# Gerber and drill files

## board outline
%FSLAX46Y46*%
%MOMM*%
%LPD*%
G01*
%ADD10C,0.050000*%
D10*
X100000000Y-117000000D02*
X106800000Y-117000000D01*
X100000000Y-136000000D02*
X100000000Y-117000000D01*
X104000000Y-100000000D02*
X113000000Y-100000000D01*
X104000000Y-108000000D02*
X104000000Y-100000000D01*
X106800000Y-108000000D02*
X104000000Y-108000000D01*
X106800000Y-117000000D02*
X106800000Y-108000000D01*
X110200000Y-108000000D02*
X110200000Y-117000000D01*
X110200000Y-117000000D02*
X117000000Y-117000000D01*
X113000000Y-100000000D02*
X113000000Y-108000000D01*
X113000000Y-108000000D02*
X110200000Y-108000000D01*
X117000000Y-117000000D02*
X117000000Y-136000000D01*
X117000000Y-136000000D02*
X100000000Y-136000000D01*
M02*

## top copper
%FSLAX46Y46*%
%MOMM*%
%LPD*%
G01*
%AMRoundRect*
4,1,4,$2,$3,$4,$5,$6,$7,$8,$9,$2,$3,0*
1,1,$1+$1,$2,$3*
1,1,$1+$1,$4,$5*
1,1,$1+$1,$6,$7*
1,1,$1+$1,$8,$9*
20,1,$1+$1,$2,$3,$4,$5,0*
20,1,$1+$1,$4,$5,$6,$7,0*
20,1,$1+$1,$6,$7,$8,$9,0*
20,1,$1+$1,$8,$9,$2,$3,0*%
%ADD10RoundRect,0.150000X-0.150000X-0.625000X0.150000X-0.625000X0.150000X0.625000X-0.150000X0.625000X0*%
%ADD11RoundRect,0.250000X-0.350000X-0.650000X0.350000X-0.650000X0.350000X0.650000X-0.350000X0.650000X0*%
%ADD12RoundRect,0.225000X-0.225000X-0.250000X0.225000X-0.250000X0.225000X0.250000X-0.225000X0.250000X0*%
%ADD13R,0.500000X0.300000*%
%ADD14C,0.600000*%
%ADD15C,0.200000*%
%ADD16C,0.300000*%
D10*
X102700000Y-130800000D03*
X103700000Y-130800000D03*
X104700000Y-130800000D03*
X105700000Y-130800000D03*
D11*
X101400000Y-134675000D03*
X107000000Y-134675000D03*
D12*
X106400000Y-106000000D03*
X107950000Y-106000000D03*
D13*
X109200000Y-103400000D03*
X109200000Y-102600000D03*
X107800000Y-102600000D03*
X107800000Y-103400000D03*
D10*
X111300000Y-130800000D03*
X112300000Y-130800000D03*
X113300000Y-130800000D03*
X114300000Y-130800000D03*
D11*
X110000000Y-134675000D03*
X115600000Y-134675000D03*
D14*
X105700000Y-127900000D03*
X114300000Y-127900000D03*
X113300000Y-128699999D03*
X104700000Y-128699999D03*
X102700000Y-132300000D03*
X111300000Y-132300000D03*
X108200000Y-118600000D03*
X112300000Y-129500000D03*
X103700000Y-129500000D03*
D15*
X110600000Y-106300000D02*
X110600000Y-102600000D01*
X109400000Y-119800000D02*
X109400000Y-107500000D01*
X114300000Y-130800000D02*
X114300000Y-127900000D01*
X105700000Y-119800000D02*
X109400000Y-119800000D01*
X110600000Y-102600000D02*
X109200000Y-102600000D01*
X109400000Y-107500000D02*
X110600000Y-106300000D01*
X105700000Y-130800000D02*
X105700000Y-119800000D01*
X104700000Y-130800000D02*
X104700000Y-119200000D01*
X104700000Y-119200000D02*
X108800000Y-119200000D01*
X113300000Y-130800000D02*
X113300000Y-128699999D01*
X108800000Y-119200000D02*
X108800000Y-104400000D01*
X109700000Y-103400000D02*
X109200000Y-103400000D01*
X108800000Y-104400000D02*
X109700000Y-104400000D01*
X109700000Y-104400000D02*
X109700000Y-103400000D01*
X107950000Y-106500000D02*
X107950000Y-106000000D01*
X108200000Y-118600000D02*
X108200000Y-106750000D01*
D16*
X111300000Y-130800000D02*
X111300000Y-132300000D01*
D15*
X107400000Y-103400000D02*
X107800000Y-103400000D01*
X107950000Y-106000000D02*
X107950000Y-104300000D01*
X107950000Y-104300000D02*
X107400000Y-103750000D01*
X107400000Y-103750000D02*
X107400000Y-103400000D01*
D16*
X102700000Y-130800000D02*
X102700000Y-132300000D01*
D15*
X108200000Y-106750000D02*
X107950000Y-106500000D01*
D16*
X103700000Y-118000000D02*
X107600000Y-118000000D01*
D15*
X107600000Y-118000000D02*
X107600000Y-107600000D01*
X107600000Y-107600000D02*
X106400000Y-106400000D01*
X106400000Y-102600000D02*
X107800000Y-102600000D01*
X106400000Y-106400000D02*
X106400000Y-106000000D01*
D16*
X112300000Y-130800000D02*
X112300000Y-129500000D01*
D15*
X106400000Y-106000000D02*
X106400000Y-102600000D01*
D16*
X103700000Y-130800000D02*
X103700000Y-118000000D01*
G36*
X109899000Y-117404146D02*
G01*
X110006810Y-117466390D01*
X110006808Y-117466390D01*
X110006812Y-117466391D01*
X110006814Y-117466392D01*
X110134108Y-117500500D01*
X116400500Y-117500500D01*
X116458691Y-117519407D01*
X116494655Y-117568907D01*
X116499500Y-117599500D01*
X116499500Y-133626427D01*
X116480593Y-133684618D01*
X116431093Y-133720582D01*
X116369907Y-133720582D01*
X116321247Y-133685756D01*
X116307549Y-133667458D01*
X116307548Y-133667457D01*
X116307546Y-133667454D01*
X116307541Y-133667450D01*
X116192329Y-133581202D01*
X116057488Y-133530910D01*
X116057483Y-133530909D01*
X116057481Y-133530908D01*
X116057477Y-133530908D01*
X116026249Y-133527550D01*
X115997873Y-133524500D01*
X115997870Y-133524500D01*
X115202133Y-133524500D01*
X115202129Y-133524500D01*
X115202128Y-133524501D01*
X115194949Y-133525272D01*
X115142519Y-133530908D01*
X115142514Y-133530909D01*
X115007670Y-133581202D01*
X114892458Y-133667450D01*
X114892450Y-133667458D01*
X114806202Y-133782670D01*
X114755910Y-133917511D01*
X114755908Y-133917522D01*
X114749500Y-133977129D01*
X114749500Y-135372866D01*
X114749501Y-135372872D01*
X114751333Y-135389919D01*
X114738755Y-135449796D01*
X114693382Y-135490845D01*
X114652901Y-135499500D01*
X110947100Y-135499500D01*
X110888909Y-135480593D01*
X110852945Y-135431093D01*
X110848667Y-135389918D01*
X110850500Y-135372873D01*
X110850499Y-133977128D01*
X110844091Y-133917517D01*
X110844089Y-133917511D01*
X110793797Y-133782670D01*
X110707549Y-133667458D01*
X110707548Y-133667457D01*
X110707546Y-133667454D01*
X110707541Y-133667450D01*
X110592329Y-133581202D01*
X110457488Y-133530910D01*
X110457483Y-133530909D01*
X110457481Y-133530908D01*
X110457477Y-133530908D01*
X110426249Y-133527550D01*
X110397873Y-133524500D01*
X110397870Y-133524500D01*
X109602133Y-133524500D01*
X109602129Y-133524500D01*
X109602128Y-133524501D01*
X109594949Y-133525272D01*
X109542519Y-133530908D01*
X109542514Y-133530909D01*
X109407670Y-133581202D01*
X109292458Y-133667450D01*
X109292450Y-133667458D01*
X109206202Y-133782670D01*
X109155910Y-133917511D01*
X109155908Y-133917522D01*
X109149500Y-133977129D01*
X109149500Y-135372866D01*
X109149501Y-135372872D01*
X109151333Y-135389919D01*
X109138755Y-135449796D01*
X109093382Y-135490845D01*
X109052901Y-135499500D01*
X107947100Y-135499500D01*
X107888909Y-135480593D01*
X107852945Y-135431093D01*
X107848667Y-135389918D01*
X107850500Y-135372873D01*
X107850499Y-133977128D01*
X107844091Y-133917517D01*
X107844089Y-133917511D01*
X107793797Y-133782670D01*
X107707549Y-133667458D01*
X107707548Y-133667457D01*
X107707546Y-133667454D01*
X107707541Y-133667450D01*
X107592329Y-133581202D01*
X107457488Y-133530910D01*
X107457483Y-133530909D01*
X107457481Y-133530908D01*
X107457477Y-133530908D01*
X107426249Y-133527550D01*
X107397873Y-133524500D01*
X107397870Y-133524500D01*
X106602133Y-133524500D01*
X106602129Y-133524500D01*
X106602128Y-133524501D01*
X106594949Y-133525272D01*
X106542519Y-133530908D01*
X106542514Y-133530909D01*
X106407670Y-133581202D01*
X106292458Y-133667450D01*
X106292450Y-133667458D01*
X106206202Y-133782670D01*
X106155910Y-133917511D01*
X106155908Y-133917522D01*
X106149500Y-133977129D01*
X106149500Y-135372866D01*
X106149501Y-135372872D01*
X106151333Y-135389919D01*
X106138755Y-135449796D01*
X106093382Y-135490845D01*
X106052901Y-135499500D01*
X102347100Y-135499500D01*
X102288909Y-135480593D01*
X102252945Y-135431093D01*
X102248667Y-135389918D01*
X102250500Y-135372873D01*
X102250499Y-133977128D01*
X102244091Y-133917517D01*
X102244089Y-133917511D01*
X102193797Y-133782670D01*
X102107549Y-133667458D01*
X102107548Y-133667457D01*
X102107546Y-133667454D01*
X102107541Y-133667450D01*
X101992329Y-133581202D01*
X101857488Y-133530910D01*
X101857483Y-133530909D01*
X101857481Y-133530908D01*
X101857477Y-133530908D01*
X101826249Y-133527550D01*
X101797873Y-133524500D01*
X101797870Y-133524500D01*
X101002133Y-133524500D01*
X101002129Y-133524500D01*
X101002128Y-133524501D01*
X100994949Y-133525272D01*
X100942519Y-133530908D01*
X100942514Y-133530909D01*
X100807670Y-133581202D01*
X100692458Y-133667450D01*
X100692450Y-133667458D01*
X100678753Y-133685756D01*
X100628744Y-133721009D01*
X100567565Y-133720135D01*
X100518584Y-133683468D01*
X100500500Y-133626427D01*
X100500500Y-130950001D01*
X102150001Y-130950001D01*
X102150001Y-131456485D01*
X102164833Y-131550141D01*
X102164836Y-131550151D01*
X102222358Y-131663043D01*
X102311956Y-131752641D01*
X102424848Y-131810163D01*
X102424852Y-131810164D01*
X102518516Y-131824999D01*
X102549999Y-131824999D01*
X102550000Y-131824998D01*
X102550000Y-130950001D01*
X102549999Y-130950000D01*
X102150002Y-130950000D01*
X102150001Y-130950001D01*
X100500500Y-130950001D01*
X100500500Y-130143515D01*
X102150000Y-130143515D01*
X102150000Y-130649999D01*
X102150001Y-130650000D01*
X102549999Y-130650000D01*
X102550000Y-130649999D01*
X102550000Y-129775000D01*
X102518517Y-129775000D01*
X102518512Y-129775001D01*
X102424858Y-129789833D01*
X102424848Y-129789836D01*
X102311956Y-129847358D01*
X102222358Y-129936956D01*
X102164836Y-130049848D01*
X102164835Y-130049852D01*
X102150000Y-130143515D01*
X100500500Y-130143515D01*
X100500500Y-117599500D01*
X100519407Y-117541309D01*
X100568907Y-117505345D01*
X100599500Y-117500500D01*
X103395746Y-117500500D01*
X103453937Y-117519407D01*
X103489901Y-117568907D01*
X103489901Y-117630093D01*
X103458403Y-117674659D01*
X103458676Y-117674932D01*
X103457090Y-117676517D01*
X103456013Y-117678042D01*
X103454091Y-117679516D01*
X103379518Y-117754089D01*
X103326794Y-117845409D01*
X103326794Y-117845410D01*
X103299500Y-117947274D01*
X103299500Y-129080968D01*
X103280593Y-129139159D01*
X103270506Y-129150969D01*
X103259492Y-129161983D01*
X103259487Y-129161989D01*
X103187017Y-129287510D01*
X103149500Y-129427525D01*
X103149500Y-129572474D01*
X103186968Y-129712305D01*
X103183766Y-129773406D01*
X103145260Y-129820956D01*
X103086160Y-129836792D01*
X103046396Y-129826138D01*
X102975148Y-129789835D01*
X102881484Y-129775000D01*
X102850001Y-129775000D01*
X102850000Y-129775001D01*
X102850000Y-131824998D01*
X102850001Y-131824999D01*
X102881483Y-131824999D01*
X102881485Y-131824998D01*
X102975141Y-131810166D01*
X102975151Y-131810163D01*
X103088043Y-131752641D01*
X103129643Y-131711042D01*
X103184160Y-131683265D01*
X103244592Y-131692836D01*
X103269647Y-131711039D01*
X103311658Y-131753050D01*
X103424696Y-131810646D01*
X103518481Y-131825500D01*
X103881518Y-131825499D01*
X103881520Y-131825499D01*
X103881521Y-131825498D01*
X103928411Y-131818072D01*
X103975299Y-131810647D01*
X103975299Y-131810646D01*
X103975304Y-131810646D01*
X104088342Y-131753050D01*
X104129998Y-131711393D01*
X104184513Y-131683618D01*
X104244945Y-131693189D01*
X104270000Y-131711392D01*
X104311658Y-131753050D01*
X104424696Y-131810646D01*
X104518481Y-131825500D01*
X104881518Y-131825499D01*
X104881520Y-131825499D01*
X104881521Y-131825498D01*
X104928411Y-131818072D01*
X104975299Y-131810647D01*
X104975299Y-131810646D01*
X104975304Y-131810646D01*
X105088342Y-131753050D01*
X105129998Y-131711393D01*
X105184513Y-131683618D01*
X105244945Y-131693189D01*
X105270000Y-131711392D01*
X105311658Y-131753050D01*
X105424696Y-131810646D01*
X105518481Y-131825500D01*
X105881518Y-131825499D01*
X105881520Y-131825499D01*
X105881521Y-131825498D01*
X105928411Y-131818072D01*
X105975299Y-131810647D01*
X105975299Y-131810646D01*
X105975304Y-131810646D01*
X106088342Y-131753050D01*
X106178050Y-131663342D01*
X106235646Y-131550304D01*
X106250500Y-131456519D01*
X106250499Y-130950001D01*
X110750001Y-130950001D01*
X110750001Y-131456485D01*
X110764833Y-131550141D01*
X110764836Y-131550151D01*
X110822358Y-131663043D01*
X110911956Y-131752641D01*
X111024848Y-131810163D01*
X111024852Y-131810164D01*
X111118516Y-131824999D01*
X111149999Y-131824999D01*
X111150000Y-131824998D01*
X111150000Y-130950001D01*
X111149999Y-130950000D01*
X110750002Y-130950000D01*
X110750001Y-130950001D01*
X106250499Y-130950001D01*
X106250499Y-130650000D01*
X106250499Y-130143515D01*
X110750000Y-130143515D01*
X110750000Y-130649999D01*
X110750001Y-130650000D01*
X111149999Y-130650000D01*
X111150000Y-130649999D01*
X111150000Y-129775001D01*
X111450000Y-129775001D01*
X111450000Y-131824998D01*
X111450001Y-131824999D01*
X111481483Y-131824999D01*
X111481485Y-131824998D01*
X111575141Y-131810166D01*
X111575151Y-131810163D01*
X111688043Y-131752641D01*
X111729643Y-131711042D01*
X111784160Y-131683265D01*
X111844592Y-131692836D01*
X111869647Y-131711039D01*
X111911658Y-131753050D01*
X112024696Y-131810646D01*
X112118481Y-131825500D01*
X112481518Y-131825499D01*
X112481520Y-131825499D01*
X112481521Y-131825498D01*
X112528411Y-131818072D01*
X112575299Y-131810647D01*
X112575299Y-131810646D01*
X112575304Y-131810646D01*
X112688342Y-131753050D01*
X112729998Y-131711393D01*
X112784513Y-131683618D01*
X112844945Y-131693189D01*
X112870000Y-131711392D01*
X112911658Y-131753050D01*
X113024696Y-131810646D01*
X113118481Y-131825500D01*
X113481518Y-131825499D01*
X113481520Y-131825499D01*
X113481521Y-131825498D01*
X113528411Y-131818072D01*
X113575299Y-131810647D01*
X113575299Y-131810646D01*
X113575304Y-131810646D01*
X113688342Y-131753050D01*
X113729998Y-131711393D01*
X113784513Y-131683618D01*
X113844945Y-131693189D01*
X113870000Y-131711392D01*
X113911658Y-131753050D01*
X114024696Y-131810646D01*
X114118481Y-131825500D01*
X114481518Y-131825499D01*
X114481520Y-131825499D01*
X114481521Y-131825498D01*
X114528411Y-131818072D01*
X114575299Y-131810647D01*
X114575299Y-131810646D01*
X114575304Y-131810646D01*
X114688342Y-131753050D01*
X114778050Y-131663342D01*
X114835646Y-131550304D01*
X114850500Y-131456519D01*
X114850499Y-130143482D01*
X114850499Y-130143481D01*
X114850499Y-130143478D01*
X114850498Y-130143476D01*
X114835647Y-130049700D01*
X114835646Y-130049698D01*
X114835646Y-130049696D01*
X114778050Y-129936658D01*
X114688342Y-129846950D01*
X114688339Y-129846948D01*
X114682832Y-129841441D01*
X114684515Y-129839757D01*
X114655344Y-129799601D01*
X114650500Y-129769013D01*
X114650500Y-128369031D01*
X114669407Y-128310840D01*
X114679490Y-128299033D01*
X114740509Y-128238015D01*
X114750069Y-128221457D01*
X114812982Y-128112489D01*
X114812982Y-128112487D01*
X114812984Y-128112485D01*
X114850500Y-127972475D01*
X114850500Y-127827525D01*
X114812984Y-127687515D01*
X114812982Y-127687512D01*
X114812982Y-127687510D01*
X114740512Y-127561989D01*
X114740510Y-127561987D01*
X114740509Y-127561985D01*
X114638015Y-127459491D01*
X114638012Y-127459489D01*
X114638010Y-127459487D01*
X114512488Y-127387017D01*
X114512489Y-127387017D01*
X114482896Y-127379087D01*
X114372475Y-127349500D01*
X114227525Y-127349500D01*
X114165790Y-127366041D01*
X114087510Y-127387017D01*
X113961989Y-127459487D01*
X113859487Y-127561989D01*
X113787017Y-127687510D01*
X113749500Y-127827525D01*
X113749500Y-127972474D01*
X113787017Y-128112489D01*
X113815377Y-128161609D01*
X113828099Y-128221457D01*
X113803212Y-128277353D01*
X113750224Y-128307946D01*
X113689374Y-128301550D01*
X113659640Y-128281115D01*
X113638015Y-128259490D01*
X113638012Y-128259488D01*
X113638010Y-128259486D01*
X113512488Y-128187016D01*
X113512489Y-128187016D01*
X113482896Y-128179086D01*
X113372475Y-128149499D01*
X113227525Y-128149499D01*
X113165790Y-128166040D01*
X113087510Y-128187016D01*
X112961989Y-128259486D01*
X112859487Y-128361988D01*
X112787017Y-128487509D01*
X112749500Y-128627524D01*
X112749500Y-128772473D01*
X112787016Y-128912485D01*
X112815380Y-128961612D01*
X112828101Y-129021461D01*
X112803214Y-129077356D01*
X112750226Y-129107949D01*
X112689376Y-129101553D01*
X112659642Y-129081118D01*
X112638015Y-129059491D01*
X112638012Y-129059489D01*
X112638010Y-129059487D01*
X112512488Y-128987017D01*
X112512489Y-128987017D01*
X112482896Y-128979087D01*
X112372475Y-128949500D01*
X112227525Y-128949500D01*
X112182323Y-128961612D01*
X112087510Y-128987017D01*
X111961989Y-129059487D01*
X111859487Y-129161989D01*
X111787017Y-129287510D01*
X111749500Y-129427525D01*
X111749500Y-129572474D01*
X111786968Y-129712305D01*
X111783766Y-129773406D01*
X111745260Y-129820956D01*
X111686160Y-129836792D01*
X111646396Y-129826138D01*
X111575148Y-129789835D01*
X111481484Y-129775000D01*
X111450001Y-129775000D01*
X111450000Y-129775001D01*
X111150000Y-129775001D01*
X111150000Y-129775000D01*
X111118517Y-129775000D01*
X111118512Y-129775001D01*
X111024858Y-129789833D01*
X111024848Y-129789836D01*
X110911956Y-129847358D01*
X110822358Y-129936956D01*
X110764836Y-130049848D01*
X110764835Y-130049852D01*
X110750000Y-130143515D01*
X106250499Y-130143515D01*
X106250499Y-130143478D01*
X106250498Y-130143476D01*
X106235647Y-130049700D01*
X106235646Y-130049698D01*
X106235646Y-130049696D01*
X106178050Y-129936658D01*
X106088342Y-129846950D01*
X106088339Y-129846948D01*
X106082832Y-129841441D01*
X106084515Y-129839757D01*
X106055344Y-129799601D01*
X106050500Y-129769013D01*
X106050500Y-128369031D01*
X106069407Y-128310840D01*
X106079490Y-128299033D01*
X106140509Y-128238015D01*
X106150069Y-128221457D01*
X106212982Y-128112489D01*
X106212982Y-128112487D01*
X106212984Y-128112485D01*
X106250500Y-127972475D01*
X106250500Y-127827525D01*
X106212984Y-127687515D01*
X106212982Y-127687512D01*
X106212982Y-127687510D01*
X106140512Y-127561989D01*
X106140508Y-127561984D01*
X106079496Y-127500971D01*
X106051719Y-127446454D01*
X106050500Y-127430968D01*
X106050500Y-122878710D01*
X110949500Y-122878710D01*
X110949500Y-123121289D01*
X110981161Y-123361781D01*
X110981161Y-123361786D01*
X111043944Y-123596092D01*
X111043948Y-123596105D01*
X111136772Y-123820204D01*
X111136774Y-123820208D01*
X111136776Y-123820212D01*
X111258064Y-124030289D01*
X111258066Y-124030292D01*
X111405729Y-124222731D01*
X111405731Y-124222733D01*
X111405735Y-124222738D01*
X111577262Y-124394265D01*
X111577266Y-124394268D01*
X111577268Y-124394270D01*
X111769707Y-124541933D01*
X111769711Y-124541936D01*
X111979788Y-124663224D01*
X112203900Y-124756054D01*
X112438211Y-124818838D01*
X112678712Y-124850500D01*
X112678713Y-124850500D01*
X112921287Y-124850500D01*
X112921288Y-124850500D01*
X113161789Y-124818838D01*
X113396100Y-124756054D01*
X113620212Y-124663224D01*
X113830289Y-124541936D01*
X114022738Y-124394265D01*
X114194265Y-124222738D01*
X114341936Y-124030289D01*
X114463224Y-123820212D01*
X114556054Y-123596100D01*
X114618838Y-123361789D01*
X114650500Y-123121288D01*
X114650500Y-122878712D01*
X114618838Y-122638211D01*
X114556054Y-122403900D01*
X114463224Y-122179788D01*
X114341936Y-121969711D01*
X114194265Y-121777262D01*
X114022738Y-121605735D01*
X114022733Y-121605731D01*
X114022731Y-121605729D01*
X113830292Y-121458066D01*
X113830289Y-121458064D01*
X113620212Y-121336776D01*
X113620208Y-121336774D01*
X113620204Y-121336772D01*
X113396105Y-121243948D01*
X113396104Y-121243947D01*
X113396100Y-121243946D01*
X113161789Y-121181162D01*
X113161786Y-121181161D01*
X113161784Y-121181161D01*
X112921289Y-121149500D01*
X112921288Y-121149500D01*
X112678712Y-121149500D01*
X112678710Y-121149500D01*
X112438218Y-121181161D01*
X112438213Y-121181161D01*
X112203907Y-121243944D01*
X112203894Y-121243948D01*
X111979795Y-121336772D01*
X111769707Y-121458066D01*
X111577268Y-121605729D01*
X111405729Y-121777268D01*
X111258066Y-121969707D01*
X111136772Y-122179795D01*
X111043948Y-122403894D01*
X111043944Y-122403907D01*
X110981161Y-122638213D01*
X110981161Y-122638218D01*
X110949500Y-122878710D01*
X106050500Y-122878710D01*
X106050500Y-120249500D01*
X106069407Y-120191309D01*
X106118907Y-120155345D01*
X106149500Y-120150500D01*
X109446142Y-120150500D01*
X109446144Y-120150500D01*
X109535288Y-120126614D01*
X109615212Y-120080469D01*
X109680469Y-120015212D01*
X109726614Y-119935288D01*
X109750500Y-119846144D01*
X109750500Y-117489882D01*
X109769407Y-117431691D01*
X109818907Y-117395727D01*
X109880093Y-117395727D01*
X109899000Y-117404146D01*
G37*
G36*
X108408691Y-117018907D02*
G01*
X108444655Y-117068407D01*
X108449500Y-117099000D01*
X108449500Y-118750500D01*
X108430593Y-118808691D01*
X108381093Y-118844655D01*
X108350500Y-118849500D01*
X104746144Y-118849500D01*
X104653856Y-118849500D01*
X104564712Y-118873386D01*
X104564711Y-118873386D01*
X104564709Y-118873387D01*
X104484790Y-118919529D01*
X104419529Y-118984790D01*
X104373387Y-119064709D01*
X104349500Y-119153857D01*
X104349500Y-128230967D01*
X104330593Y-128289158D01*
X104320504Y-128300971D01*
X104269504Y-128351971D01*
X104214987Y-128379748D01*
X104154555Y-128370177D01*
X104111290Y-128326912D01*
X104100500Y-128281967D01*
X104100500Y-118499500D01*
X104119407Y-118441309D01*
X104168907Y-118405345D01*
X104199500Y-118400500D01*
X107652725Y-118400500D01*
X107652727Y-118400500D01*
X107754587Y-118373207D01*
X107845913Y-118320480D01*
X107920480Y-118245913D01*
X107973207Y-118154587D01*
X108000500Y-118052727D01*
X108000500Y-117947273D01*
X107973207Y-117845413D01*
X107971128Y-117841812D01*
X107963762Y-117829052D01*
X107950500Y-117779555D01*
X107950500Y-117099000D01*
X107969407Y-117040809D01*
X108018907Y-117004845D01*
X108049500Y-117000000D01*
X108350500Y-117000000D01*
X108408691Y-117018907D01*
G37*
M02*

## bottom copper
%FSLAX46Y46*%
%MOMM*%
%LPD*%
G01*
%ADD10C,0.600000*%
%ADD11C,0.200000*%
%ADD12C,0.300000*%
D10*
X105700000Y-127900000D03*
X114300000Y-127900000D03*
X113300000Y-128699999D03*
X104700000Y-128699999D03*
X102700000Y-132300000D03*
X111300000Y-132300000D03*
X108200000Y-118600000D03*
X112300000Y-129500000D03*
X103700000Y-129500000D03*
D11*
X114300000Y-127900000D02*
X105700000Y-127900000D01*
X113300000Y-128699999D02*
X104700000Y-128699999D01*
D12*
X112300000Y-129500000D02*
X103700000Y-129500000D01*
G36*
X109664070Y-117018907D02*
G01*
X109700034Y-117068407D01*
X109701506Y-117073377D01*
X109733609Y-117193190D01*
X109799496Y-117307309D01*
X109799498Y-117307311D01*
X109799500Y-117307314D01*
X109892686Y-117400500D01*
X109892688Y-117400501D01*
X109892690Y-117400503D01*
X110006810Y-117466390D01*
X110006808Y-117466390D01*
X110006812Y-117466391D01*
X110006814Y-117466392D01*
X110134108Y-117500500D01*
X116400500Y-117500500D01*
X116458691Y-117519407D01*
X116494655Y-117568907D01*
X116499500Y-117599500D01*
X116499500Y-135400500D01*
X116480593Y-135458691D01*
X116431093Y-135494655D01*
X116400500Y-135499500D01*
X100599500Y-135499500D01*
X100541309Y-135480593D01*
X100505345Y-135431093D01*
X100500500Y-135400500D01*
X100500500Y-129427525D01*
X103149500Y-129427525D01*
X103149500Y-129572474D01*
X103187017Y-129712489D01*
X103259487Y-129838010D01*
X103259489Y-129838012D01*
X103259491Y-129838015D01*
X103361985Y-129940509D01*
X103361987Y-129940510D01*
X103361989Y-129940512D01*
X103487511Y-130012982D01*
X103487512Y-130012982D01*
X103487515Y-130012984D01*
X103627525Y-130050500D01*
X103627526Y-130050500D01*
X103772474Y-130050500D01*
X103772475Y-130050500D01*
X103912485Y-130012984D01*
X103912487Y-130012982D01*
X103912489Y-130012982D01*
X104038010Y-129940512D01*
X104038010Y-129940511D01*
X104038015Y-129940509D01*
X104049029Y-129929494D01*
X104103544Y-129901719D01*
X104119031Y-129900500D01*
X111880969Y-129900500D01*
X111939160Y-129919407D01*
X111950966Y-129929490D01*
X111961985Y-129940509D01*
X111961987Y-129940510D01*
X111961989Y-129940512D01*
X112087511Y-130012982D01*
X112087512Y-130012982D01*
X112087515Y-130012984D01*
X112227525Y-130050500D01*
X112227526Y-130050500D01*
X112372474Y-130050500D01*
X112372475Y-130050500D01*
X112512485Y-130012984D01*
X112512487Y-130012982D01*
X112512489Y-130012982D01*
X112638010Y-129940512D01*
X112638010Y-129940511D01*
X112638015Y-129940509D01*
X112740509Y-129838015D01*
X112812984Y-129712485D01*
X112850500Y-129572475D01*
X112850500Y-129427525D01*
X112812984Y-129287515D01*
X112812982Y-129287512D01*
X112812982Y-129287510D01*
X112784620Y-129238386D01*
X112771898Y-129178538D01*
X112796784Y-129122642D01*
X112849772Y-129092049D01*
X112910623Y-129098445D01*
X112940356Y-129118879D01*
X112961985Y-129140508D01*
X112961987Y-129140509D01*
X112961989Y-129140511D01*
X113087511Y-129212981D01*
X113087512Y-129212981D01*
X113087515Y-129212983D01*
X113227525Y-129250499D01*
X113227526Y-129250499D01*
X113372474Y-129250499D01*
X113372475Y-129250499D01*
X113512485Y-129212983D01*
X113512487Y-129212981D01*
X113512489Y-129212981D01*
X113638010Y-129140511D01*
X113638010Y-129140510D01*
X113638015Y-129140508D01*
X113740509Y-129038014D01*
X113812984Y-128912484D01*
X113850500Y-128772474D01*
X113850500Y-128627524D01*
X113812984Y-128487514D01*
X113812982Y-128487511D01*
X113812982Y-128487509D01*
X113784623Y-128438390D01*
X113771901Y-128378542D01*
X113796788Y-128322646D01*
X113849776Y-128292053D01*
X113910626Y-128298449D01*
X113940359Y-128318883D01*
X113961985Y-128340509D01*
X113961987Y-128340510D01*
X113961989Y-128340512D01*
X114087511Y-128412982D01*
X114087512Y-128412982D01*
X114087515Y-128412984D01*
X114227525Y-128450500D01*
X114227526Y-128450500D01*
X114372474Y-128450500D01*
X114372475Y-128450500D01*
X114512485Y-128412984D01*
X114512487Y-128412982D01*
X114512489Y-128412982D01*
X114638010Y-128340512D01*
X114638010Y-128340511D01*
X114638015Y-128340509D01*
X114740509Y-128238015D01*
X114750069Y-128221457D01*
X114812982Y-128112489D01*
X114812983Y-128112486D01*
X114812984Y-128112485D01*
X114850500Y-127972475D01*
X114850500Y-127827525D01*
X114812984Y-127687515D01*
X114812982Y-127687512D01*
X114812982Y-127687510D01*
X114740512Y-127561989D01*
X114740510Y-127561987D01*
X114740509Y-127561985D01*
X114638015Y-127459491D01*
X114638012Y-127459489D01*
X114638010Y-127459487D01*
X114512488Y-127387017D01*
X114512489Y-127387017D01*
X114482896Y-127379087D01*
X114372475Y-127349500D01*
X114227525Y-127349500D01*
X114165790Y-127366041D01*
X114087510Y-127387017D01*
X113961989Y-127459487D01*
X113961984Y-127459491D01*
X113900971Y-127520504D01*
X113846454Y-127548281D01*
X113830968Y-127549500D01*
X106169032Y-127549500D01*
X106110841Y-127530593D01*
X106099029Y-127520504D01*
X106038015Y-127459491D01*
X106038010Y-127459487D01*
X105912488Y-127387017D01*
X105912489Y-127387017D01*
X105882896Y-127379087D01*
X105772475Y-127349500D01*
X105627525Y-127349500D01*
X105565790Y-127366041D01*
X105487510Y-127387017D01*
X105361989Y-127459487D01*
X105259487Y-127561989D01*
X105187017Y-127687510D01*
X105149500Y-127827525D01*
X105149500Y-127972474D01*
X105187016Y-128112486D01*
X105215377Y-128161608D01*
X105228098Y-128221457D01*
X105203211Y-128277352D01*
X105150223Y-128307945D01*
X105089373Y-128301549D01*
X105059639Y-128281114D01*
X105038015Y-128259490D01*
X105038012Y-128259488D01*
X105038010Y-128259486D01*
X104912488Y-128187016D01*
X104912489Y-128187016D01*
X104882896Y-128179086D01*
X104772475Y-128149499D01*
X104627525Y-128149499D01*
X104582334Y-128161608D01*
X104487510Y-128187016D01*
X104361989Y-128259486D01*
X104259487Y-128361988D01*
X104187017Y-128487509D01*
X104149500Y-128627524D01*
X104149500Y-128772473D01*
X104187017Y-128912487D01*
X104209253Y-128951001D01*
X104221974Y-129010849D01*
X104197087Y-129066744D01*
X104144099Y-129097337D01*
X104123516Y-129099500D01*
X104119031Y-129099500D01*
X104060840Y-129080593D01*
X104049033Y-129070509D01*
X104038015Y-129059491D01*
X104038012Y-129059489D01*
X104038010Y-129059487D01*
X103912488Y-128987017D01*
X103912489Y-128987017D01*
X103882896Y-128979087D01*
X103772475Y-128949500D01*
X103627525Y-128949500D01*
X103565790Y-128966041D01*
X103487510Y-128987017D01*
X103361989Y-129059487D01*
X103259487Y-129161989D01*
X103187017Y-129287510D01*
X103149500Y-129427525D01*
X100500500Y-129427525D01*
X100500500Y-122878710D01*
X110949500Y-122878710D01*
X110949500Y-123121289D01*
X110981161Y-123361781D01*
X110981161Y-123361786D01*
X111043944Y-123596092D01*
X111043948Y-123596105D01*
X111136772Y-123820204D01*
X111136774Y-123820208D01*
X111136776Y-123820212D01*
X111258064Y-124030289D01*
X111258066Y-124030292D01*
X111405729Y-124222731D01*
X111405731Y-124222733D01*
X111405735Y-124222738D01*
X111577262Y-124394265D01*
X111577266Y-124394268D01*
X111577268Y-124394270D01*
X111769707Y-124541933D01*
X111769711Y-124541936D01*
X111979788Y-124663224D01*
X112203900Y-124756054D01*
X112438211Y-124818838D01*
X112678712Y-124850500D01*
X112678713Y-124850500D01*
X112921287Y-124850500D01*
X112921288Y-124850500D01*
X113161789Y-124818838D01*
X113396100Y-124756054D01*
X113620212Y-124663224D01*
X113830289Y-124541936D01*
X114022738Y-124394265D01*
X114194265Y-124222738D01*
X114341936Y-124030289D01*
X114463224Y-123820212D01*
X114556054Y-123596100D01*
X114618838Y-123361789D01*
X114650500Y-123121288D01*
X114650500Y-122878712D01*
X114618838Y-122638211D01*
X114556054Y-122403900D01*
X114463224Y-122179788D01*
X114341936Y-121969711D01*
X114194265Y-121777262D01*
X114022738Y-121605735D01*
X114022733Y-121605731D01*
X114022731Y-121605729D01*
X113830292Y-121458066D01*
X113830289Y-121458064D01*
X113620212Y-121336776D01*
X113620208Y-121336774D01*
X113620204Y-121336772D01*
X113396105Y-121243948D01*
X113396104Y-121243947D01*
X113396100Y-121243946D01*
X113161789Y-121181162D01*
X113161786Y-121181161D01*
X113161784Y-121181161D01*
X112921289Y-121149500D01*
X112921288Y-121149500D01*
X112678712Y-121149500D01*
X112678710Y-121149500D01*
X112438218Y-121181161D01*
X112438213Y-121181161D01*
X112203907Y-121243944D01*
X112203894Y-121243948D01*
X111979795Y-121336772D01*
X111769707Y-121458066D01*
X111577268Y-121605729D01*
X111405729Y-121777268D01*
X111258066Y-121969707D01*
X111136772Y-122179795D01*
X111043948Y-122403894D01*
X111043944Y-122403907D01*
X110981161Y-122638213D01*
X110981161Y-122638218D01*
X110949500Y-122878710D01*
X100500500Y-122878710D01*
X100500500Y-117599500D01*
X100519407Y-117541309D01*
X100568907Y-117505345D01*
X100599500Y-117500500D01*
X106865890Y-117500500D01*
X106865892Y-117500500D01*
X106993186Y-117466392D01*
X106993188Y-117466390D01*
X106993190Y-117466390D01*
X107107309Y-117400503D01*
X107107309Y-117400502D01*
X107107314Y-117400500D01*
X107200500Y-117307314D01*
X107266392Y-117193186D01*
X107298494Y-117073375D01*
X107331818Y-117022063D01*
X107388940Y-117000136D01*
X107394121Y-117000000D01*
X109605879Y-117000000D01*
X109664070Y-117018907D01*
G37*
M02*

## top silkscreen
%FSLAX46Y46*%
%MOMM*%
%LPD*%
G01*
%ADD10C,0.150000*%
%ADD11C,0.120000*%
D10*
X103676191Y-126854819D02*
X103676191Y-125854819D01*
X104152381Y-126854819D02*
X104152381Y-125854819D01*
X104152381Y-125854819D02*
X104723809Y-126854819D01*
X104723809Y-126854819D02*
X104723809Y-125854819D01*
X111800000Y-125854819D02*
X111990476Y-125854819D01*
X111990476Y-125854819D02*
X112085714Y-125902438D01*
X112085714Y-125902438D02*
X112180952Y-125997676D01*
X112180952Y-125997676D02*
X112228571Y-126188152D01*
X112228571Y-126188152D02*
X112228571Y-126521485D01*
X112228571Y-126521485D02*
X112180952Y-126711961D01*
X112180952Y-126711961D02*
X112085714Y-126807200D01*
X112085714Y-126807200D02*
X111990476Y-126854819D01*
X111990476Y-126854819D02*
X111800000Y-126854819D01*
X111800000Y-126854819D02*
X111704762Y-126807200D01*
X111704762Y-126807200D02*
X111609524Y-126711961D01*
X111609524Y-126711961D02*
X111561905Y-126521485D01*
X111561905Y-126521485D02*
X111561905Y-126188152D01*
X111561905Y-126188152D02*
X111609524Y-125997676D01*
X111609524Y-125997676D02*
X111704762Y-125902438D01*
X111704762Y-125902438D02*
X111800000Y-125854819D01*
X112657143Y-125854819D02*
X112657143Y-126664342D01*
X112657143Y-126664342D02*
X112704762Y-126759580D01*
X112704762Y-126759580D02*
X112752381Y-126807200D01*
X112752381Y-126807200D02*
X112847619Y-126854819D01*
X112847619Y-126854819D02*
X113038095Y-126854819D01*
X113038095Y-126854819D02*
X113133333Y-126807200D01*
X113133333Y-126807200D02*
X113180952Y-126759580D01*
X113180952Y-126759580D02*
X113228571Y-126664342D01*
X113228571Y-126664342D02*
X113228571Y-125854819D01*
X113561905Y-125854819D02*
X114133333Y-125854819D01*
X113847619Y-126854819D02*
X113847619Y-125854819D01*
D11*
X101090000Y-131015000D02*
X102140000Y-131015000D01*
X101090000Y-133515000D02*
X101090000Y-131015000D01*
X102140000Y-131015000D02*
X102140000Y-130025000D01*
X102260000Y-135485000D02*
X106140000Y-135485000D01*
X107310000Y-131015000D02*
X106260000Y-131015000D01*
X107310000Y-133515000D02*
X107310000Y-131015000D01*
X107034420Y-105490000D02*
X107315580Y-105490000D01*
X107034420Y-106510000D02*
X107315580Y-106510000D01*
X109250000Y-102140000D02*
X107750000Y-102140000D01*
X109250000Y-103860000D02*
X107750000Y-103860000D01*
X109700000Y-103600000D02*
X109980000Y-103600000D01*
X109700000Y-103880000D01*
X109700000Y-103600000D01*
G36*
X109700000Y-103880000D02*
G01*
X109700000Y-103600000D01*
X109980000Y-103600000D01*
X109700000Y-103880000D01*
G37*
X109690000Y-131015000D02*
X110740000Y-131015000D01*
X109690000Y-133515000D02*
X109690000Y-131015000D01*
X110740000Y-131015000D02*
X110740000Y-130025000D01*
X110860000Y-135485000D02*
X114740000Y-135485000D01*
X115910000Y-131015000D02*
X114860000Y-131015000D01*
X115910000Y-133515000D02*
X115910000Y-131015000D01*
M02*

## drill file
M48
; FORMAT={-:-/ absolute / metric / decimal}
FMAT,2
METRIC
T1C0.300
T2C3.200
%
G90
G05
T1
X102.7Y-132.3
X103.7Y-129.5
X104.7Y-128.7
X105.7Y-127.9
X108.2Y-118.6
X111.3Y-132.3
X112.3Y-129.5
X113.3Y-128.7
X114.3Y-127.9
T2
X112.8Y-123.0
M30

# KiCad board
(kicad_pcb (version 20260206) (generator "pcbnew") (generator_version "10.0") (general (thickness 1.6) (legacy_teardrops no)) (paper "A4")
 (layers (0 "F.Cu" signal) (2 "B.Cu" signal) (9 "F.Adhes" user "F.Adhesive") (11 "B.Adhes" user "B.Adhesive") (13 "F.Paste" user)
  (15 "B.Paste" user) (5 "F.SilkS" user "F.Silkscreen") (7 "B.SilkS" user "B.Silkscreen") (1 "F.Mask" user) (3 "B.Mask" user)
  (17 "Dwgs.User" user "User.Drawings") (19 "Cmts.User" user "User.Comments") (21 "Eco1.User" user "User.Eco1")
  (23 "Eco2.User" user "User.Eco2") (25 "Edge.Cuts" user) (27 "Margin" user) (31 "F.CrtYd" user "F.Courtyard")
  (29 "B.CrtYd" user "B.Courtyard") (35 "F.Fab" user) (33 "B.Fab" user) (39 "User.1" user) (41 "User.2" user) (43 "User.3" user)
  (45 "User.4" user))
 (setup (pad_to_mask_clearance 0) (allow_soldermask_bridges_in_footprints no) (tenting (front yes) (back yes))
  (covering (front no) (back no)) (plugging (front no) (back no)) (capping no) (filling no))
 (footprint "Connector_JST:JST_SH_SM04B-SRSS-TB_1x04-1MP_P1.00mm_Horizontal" (layer "F.Cu") (at 104.2 132.8)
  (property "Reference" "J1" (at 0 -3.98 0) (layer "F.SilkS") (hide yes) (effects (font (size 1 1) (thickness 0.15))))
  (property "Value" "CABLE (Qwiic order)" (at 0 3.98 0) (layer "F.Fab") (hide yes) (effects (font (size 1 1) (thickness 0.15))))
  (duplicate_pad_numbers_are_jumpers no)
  (fp_line (start -3.11 -1.785) (end -2.06 -1.785) (stroke (width 0.12) (type solid)) (layer "F.SilkS"))
  (fp_line (start -3.11 0.715) (end -3.11 -1.785) (stroke (width 0.12) (type solid)) (layer "F.SilkS"))
  (fp_line (start -2.06 -1.785) (end -2.06 -2.775) (stroke (width 0.12) (type solid)) (layer "F.SilkS"))
  (fp_line (start -1.94 2.685) (end 1.94 2.685) (stroke (width 0.12) (type solid)) (layer "F.SilkS"))
  (fp_line (start 3.11 -1.785) (end 2.06 -1.785) (stroke (width 0.12) (type solid)) (layer "F.SilkS"))
  (fp_line (start 3.11 0.715) (end 3.11 -1.785) (stroke (width 0.12) (type solid)) (layer "F.SilkS"))
  (pad "1" smd roundrect (at -1.5 -2) (size 0.6 1.55) (layers "F.Cu" "F.Mask" "F.Paste") (roundrect_rratio 0.25) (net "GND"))
  (pad "2" smd roundrect (at -0.5 -2) (size 0.6 1.55) (layers "F.Cu" "F.Mask" "F.Paste") (roundrect_rratio 0.25) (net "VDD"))
  (pad "3" smd roundrect (at 0.5 -2) (size 0.6 1.55) (layers "F.Cu" "F.Mask" "F.Paste") (roundrect_rratio 0.25) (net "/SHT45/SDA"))
  (pad "4" smd roundrect (at 1.5 -2) (size 0.6 1.55) (layers "F.Cu" "F.Mask" "F.Paste") (roundrect_rratio 0.25) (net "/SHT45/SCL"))
  (pad "MP" smd roundrect (at -2.8 1.875) (size 1.2 1.8) (layers "F.Cu" "F.Mask" "F.Paste") (roundrect_rratio 0.208333))
  (pad "MP" smd roundrect (at 2.8 1.875) (size 1.2 1.8) (layers "F.Cu" "F.Mask" "F.Paste") (roundrect_rratio 0.208333)))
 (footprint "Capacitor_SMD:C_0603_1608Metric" (layer "F.Cu") (at 107.175 106)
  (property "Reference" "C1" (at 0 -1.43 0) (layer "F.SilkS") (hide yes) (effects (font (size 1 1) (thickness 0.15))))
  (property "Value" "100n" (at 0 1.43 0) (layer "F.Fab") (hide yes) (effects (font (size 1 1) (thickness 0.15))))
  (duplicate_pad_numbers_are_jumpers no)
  (fp_line (start -0.14058 -0.51) (end 0.14058 -0.51) (stroke (width 0.12) (type solid)) (layer "F.SilkS"))
  (fp_line (start -0.14058 0.51) (end 0.14058 0.51) (stroke (width 0.12) (type solid)) (layer "F.SilkS"))
  (pad "1" smd roundrect (at -0.775 0) (size 0.9 0.95) (layers "F.Cu" "F.Mask" "F.Paste") (roundrect_rratio 0.25) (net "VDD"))
  (pad "2" smd roundrect (at 0.775 0) (size 0.9 0.95) (layers "F.Cu" "F.Mask" "F.Paste") (roundrect_rratio 0.25) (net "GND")))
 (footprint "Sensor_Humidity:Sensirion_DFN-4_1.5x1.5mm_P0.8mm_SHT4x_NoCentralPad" (layer "F.Cu") (at 108.5 103 180)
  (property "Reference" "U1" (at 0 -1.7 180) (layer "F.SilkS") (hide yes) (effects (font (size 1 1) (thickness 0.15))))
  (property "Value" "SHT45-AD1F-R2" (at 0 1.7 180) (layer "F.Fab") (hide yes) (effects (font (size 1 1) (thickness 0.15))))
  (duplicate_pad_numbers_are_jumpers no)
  (fp_line (start -0.75 0.86) (end 0.75 0.86) (stroke (width 0.12) (type solid)) (layer "F.SilkS"))
  (fp_line (start -0.75 -0.86) (end 0.75 -0.86) (stroke (width 0.12) (type solid)) (layer "F.SilkS"))
  (fp_poly
   (pts (xy -1.2 -0.6) (xy -1.48 -0.6) (xy -1.2 -0.88) (xy -1.2 -0.6)) (stroke (width 0.12) (type solid)) (fill yes) (layer "F.SilkS"))
  (pad "1" smd rect (at -0.7 -0.4 180) (size 0.5 0.3) (layers "F.Cu" "F.Mask" "F.Paste") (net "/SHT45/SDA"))
  (pad "2" smd rect (at -0.7 0.4 180) (size 0.5 0.3) (layers "F.Cu" "F.Mask" "F.Paste") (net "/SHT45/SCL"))
  (pad "3" smd rect (at 0.7 0.4 180) (size 0.5 0.3) (layers "F.Cu" "F.Mask" "F.Paste") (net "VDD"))
  (pad "4" smd rect (at 0.7 -0.4 180) (size 0.5 0.3) (layers "F.Cu" "F.Mask" "F.Paste") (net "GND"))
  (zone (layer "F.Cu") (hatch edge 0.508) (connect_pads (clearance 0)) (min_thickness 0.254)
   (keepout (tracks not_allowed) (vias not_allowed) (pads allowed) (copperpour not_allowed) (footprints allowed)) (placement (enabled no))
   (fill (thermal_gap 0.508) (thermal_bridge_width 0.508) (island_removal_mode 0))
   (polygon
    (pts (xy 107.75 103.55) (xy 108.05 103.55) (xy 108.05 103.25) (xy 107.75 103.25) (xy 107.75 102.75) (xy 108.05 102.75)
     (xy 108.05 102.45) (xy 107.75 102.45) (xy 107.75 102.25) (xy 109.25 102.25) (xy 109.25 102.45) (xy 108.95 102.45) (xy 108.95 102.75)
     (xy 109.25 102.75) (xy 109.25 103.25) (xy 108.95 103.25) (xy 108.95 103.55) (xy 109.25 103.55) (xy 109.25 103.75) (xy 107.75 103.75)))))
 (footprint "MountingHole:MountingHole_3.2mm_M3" (layer "F.Cu") (at 112.8 123)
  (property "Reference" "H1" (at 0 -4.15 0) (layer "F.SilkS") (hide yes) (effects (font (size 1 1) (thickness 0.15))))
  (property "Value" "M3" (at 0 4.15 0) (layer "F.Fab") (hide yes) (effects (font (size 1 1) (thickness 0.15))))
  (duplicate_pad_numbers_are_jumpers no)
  (pad "" np_thru_hole circle (at 0 0) (size 3.2 3.2) (drill 3.2) (layers "*.Cu" "*.Mask")))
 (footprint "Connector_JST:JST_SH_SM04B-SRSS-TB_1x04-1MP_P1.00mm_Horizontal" (layer "F.Cu") (at 112.8 132.8)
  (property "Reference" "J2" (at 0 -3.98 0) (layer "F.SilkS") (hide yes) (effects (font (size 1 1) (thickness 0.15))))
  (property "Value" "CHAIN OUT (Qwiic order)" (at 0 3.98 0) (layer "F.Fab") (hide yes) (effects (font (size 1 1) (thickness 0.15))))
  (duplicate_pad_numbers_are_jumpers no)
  (fp_line (start -3.11 -1.785) (end -2.06 -1.785) (stroke (width 0.12) (type solid)) (layer "F.SilkS"))
  (fp_line (start -3.11 0.715) (end -3.11 -1.785) (stroke (width 0.12) (type solid)) (layer "F.SilkS"))
  (fp_line (start -2.06 -1.785) (end -2.06 -2.775) (stroke (width 0.12) (type solid)) (layer "F.SilkS"))
  (fp_line (start -1.94 2.685) (end 1.94 2.685) (stroke (width 0.12) (type solid)) (layer "F.SilkS"))
  (fp_line (start 3.11 -1.785) (end 2.06 -1.785) (stroke (width 0.12) (type solid)) (layer "F.SilkS"))
  (fp_line (start 3.11 0.715) (end 3.11 -1.785) (stroke (width 0.12) (type solid)) (layer "F.SilkS"))
  (pad "1" smd roundrect (at -1.5 -2) (size 0.6 1.55) (layers "F.Cu" "F.Mask" "F.Paste") (roundrect_rratio 0.25) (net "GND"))
  (pad "2" smd roundrect (at -0.5 -2) (size 0.6 1.55) (layers "F.Cu" "F.Mask" "F.Paste") (roundrect_rratio 0.25) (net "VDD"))
  (pad "3" smd roundrect (at 0.5 -2) (size 0.6 1.55) (layers "F.Cu" "F.Mask" "F.Paste") (roundrect_rratio 0.25) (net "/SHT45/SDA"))
  (pad "4" smd roundrect (at 1.5 -2) (size 0.6 1.55) (layers "F.Cu" "F.Mask" "F.Paste") (roundrect_rratio 0.25) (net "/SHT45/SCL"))
  (pad "MP" smd roundrect (at -2.8 1.875) (size 1.2 1.8) (layers "F.Cu" "F.Mask" "F.Paste") (roundrect_rratio 0.208333))
  (pad "MP" smd roundrect (at 2.8 1.875) (size 1.2 1.8) (layers "F.Cu" "F.Mask" "F.Paste") (roundrect_rratio 0.208333)))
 (gr_line (start 100 117) (end 106.8 117) (stroke (width 0.05) (type default)) (layer "Edge.Cuts"))
 (gr_line (start 100 136) (end 100 117) (stroke (width 0.05) (type default)) (layer "Edge.Cuts"))
 (gr_line (start 104 100) (end 113 100) (stroke (width 0.05) (type default)) (layer "Edge.Cuts"))
 (gr_line (start 104 108) (end 104 100) (stroke (width 0.05) (type default)) (layer "Edge.Cuts"))
 (gr_line (start 106.8 108) (end 104 108) (stroke (width 0.05) (type default)) (layer "Edge.Cuts"))
 (gr_line (start 106.8 117) (end 106.8 108) (stroke (width 0.05) (type default)) (layer "Edge.Cuts"))
 (gr_line (start 110.2 108) (end 110.2 117) (stroke (width 0.05) (type default)) (layer "Edge.Cuts"))
 (gr_line (start 110.2 117) (end 117 117) (stroke (width 0.05) (type default)) (layer "Edge.Cuts"))
 (gr_line (start 113 100) (end 113 108) (stroke (width 0.05) (type default)) (layer "Edge.Cuts"))
 (gr_line (start 113 108) (end 110.2 108) (stroke (width 0.05) (type default)) (layer "Edge.Cuts"))
 (gr_line (start 117 117) (end 117 136) (stroke (width 0.05) (type default)) (layer "Edge.Cuts"))
 (gr_line (start 117 136) (end 100 136) (stroke (width 0.05) (type default)) (layer "Edge.Cuts"))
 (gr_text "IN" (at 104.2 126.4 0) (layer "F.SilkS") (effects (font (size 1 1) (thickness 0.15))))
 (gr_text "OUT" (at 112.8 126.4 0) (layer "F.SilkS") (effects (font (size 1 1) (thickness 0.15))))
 (segment (start 110.6 106.3) (end 110.6 102.6) (width 0.2) (layer "F.Cu") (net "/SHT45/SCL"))
 (segment (start 109.4 119.8) (end 109.4 107.5) (width 0.2) (layer "F.Cu") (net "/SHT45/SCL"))
 (segment (start 114.3 130.8) (end 114.3 127.9) (width 0.2) (layer "F.Cu") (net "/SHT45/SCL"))
 (segment (start 105.7 119.8) (end 109.4 119.8) (width 0.2) (layer "F.Cu") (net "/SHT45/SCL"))
 (segment (start 110.6 102.6) (end 109.2 102.6) (width 0.2) (layer "F.Cu") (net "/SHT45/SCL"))
 (segment (start 109.4 107.5) (end 110.6 106.3) (width 0.2) (layer "F.Cu") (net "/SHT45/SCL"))
 (segment (start 105.7 130.8) (end 105.7 119.8) (width 0.2) (layer "F.Cu") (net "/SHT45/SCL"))
 (via (at 105.7 127.9) (size 0.6) (drill 0.3) (layers "F.Cu" "B.Cu") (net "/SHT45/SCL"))
 (via (at 114.3 127.9) (size 0.6) (drill 0.3) (layers "F.Cu" "B.Cu") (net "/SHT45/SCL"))
 (segment (start 114.3 127.9) (end 105.7 127.9) (width 0.2) (layer "B.Cu") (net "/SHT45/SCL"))
 (segment (start 104.7 130.8) (end 104.7 119.2) (width 0.2) (layer "F.Cu") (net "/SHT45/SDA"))
 (segment (start 104.7 119.2) (end 108.8 119.2) (width 0.2) (layer "F.Cu") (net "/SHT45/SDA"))
 (segment (start 113.3 130.8) (end 113.3 128.699999) (width 0.2) (layer "F.Cu") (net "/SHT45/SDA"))
 (segment (start 108.8 119.2) (end 108.8 104.4) (width 0.2) (layer "F.Cu") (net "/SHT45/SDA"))
 (segment (start 109.7 103.4) (end 109.2 103.4) (width 0.2) (layer "F.Cu") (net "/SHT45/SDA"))
 (segment (start 108.8 104.4) (end 109.7 104.4) (width 0.2) (layer "F.Cu") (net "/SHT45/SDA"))
 (segment (start 109.7 104.4) (end 109.7 103.4) (width 0.2) (layer "F.Cu") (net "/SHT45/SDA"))
 (via (at 113.3 128.699999) (size 0.6) (drill 0.3) (layers "F.Cu" "B.Cu") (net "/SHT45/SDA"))
 (via (at 104.7 128.699999) (size 0.6) (drill 0.3) (layers "F.Cu" "B.Cu") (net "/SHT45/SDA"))
 (segment (start 113.3 128.699999) (end 104.7 128.699999) (width 0.2) (layer "B.Cu") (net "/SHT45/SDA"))
 (segment (start 107.95 106.5) (end 107.95 106) (width 0.2) (layer "F.Cu") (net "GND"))
 (segment (start 108.2 118.6) (end 108.2 106.75) (width 0.2) (layer "F.Cu") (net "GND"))
 (segment (start 111.3 130.8) (end 111.3 132.3) (width 0.3) (layer "F.Cu") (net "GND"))
 (segment (start 107.4 103.4) (end 107.8 103.4) (width 0.2) (layer "F.Cu") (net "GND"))
 (segment (start 107.95 106) (end 107.95 104.3) (width 0.2) (layer "F.Cu") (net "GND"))
 (segment (start 107.95 104.3) (end 107.4 103.75) (width 0.2) (layer "F.Cu") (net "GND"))
 (segment (start 107.4 103.75) (end 107.4 103.4) (width 0.2) (layer "F.Cu") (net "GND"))
 (segment (start 102.7 130.8) (end 102.7 132.3) (width 0.3) (layer "F.Cu") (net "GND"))
 (segment (start 108.2 106.75) (end 107.95 106.5) (width 0.2) (layer "F.Cu") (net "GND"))
 (via (at 102.7 132.3) (size 0.6) (drill 0.3) (layers "F.Cu" "B.Cu") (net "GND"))
 (via (at 111.3 132.3) (size 0.6) (drill 0.3) (layers "F.Cu" "B.Cu") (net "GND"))
 (via (at 108.2 118.6) (size 0.6) (drill 0.3) (layers "F.Cu" "B.Cu") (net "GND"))
 (segment (start 103.7 118) (end 107.6 118) (width 0.3) (layer "F.Cu") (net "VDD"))
 (segment (start 107.6 118) (end 107.6 107.6) (width 0.2) (layer "F.Cu") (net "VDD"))
 (segment (start 107.6 107.6) (end 106.4 106.4) (width 0.2) (layer "F.Cu") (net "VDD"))
 (segment (start 106.4 102.6) (end 107.8 102.6) (width 0.2) (layer "F.Cu") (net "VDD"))
 (segment (start 106.4 106.4) (end 106.4 106) (width 0.2) (layer "F.Cu") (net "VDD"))
 (segment (start 112.3 130.8) (end 112.3 129.5) (width 0.3) (layer "F.Cu") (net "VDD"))
 (segment (start 106.4 106) (end 106.4 102.6) (width 0.2) (layer "F.Cu") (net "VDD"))
 (segment (start 103.7 130.8) (end 103.7 118) (width 0.3) (layer "F.Cu") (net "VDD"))
 (via (at 112.3 129.5) (size 0.6) (drill 0.3) (layers "F.Cu" "B.Cu") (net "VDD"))
 (via (at 103.7 129.5) (size 0.6) (drill 0.3) (layers "F.Cu" "B.Cu") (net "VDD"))
 (segment (start 112.3 129.5) (end 103.7 129.5) (width 0.3) (layer "B.Cu") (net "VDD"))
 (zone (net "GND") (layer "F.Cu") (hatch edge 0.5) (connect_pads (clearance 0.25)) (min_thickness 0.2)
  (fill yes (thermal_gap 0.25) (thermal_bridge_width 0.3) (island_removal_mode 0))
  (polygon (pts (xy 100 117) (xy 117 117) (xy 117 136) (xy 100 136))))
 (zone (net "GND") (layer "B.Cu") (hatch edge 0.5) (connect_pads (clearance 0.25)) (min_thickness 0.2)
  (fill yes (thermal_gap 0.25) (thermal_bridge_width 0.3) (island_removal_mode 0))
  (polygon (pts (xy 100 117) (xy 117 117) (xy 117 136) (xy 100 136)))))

